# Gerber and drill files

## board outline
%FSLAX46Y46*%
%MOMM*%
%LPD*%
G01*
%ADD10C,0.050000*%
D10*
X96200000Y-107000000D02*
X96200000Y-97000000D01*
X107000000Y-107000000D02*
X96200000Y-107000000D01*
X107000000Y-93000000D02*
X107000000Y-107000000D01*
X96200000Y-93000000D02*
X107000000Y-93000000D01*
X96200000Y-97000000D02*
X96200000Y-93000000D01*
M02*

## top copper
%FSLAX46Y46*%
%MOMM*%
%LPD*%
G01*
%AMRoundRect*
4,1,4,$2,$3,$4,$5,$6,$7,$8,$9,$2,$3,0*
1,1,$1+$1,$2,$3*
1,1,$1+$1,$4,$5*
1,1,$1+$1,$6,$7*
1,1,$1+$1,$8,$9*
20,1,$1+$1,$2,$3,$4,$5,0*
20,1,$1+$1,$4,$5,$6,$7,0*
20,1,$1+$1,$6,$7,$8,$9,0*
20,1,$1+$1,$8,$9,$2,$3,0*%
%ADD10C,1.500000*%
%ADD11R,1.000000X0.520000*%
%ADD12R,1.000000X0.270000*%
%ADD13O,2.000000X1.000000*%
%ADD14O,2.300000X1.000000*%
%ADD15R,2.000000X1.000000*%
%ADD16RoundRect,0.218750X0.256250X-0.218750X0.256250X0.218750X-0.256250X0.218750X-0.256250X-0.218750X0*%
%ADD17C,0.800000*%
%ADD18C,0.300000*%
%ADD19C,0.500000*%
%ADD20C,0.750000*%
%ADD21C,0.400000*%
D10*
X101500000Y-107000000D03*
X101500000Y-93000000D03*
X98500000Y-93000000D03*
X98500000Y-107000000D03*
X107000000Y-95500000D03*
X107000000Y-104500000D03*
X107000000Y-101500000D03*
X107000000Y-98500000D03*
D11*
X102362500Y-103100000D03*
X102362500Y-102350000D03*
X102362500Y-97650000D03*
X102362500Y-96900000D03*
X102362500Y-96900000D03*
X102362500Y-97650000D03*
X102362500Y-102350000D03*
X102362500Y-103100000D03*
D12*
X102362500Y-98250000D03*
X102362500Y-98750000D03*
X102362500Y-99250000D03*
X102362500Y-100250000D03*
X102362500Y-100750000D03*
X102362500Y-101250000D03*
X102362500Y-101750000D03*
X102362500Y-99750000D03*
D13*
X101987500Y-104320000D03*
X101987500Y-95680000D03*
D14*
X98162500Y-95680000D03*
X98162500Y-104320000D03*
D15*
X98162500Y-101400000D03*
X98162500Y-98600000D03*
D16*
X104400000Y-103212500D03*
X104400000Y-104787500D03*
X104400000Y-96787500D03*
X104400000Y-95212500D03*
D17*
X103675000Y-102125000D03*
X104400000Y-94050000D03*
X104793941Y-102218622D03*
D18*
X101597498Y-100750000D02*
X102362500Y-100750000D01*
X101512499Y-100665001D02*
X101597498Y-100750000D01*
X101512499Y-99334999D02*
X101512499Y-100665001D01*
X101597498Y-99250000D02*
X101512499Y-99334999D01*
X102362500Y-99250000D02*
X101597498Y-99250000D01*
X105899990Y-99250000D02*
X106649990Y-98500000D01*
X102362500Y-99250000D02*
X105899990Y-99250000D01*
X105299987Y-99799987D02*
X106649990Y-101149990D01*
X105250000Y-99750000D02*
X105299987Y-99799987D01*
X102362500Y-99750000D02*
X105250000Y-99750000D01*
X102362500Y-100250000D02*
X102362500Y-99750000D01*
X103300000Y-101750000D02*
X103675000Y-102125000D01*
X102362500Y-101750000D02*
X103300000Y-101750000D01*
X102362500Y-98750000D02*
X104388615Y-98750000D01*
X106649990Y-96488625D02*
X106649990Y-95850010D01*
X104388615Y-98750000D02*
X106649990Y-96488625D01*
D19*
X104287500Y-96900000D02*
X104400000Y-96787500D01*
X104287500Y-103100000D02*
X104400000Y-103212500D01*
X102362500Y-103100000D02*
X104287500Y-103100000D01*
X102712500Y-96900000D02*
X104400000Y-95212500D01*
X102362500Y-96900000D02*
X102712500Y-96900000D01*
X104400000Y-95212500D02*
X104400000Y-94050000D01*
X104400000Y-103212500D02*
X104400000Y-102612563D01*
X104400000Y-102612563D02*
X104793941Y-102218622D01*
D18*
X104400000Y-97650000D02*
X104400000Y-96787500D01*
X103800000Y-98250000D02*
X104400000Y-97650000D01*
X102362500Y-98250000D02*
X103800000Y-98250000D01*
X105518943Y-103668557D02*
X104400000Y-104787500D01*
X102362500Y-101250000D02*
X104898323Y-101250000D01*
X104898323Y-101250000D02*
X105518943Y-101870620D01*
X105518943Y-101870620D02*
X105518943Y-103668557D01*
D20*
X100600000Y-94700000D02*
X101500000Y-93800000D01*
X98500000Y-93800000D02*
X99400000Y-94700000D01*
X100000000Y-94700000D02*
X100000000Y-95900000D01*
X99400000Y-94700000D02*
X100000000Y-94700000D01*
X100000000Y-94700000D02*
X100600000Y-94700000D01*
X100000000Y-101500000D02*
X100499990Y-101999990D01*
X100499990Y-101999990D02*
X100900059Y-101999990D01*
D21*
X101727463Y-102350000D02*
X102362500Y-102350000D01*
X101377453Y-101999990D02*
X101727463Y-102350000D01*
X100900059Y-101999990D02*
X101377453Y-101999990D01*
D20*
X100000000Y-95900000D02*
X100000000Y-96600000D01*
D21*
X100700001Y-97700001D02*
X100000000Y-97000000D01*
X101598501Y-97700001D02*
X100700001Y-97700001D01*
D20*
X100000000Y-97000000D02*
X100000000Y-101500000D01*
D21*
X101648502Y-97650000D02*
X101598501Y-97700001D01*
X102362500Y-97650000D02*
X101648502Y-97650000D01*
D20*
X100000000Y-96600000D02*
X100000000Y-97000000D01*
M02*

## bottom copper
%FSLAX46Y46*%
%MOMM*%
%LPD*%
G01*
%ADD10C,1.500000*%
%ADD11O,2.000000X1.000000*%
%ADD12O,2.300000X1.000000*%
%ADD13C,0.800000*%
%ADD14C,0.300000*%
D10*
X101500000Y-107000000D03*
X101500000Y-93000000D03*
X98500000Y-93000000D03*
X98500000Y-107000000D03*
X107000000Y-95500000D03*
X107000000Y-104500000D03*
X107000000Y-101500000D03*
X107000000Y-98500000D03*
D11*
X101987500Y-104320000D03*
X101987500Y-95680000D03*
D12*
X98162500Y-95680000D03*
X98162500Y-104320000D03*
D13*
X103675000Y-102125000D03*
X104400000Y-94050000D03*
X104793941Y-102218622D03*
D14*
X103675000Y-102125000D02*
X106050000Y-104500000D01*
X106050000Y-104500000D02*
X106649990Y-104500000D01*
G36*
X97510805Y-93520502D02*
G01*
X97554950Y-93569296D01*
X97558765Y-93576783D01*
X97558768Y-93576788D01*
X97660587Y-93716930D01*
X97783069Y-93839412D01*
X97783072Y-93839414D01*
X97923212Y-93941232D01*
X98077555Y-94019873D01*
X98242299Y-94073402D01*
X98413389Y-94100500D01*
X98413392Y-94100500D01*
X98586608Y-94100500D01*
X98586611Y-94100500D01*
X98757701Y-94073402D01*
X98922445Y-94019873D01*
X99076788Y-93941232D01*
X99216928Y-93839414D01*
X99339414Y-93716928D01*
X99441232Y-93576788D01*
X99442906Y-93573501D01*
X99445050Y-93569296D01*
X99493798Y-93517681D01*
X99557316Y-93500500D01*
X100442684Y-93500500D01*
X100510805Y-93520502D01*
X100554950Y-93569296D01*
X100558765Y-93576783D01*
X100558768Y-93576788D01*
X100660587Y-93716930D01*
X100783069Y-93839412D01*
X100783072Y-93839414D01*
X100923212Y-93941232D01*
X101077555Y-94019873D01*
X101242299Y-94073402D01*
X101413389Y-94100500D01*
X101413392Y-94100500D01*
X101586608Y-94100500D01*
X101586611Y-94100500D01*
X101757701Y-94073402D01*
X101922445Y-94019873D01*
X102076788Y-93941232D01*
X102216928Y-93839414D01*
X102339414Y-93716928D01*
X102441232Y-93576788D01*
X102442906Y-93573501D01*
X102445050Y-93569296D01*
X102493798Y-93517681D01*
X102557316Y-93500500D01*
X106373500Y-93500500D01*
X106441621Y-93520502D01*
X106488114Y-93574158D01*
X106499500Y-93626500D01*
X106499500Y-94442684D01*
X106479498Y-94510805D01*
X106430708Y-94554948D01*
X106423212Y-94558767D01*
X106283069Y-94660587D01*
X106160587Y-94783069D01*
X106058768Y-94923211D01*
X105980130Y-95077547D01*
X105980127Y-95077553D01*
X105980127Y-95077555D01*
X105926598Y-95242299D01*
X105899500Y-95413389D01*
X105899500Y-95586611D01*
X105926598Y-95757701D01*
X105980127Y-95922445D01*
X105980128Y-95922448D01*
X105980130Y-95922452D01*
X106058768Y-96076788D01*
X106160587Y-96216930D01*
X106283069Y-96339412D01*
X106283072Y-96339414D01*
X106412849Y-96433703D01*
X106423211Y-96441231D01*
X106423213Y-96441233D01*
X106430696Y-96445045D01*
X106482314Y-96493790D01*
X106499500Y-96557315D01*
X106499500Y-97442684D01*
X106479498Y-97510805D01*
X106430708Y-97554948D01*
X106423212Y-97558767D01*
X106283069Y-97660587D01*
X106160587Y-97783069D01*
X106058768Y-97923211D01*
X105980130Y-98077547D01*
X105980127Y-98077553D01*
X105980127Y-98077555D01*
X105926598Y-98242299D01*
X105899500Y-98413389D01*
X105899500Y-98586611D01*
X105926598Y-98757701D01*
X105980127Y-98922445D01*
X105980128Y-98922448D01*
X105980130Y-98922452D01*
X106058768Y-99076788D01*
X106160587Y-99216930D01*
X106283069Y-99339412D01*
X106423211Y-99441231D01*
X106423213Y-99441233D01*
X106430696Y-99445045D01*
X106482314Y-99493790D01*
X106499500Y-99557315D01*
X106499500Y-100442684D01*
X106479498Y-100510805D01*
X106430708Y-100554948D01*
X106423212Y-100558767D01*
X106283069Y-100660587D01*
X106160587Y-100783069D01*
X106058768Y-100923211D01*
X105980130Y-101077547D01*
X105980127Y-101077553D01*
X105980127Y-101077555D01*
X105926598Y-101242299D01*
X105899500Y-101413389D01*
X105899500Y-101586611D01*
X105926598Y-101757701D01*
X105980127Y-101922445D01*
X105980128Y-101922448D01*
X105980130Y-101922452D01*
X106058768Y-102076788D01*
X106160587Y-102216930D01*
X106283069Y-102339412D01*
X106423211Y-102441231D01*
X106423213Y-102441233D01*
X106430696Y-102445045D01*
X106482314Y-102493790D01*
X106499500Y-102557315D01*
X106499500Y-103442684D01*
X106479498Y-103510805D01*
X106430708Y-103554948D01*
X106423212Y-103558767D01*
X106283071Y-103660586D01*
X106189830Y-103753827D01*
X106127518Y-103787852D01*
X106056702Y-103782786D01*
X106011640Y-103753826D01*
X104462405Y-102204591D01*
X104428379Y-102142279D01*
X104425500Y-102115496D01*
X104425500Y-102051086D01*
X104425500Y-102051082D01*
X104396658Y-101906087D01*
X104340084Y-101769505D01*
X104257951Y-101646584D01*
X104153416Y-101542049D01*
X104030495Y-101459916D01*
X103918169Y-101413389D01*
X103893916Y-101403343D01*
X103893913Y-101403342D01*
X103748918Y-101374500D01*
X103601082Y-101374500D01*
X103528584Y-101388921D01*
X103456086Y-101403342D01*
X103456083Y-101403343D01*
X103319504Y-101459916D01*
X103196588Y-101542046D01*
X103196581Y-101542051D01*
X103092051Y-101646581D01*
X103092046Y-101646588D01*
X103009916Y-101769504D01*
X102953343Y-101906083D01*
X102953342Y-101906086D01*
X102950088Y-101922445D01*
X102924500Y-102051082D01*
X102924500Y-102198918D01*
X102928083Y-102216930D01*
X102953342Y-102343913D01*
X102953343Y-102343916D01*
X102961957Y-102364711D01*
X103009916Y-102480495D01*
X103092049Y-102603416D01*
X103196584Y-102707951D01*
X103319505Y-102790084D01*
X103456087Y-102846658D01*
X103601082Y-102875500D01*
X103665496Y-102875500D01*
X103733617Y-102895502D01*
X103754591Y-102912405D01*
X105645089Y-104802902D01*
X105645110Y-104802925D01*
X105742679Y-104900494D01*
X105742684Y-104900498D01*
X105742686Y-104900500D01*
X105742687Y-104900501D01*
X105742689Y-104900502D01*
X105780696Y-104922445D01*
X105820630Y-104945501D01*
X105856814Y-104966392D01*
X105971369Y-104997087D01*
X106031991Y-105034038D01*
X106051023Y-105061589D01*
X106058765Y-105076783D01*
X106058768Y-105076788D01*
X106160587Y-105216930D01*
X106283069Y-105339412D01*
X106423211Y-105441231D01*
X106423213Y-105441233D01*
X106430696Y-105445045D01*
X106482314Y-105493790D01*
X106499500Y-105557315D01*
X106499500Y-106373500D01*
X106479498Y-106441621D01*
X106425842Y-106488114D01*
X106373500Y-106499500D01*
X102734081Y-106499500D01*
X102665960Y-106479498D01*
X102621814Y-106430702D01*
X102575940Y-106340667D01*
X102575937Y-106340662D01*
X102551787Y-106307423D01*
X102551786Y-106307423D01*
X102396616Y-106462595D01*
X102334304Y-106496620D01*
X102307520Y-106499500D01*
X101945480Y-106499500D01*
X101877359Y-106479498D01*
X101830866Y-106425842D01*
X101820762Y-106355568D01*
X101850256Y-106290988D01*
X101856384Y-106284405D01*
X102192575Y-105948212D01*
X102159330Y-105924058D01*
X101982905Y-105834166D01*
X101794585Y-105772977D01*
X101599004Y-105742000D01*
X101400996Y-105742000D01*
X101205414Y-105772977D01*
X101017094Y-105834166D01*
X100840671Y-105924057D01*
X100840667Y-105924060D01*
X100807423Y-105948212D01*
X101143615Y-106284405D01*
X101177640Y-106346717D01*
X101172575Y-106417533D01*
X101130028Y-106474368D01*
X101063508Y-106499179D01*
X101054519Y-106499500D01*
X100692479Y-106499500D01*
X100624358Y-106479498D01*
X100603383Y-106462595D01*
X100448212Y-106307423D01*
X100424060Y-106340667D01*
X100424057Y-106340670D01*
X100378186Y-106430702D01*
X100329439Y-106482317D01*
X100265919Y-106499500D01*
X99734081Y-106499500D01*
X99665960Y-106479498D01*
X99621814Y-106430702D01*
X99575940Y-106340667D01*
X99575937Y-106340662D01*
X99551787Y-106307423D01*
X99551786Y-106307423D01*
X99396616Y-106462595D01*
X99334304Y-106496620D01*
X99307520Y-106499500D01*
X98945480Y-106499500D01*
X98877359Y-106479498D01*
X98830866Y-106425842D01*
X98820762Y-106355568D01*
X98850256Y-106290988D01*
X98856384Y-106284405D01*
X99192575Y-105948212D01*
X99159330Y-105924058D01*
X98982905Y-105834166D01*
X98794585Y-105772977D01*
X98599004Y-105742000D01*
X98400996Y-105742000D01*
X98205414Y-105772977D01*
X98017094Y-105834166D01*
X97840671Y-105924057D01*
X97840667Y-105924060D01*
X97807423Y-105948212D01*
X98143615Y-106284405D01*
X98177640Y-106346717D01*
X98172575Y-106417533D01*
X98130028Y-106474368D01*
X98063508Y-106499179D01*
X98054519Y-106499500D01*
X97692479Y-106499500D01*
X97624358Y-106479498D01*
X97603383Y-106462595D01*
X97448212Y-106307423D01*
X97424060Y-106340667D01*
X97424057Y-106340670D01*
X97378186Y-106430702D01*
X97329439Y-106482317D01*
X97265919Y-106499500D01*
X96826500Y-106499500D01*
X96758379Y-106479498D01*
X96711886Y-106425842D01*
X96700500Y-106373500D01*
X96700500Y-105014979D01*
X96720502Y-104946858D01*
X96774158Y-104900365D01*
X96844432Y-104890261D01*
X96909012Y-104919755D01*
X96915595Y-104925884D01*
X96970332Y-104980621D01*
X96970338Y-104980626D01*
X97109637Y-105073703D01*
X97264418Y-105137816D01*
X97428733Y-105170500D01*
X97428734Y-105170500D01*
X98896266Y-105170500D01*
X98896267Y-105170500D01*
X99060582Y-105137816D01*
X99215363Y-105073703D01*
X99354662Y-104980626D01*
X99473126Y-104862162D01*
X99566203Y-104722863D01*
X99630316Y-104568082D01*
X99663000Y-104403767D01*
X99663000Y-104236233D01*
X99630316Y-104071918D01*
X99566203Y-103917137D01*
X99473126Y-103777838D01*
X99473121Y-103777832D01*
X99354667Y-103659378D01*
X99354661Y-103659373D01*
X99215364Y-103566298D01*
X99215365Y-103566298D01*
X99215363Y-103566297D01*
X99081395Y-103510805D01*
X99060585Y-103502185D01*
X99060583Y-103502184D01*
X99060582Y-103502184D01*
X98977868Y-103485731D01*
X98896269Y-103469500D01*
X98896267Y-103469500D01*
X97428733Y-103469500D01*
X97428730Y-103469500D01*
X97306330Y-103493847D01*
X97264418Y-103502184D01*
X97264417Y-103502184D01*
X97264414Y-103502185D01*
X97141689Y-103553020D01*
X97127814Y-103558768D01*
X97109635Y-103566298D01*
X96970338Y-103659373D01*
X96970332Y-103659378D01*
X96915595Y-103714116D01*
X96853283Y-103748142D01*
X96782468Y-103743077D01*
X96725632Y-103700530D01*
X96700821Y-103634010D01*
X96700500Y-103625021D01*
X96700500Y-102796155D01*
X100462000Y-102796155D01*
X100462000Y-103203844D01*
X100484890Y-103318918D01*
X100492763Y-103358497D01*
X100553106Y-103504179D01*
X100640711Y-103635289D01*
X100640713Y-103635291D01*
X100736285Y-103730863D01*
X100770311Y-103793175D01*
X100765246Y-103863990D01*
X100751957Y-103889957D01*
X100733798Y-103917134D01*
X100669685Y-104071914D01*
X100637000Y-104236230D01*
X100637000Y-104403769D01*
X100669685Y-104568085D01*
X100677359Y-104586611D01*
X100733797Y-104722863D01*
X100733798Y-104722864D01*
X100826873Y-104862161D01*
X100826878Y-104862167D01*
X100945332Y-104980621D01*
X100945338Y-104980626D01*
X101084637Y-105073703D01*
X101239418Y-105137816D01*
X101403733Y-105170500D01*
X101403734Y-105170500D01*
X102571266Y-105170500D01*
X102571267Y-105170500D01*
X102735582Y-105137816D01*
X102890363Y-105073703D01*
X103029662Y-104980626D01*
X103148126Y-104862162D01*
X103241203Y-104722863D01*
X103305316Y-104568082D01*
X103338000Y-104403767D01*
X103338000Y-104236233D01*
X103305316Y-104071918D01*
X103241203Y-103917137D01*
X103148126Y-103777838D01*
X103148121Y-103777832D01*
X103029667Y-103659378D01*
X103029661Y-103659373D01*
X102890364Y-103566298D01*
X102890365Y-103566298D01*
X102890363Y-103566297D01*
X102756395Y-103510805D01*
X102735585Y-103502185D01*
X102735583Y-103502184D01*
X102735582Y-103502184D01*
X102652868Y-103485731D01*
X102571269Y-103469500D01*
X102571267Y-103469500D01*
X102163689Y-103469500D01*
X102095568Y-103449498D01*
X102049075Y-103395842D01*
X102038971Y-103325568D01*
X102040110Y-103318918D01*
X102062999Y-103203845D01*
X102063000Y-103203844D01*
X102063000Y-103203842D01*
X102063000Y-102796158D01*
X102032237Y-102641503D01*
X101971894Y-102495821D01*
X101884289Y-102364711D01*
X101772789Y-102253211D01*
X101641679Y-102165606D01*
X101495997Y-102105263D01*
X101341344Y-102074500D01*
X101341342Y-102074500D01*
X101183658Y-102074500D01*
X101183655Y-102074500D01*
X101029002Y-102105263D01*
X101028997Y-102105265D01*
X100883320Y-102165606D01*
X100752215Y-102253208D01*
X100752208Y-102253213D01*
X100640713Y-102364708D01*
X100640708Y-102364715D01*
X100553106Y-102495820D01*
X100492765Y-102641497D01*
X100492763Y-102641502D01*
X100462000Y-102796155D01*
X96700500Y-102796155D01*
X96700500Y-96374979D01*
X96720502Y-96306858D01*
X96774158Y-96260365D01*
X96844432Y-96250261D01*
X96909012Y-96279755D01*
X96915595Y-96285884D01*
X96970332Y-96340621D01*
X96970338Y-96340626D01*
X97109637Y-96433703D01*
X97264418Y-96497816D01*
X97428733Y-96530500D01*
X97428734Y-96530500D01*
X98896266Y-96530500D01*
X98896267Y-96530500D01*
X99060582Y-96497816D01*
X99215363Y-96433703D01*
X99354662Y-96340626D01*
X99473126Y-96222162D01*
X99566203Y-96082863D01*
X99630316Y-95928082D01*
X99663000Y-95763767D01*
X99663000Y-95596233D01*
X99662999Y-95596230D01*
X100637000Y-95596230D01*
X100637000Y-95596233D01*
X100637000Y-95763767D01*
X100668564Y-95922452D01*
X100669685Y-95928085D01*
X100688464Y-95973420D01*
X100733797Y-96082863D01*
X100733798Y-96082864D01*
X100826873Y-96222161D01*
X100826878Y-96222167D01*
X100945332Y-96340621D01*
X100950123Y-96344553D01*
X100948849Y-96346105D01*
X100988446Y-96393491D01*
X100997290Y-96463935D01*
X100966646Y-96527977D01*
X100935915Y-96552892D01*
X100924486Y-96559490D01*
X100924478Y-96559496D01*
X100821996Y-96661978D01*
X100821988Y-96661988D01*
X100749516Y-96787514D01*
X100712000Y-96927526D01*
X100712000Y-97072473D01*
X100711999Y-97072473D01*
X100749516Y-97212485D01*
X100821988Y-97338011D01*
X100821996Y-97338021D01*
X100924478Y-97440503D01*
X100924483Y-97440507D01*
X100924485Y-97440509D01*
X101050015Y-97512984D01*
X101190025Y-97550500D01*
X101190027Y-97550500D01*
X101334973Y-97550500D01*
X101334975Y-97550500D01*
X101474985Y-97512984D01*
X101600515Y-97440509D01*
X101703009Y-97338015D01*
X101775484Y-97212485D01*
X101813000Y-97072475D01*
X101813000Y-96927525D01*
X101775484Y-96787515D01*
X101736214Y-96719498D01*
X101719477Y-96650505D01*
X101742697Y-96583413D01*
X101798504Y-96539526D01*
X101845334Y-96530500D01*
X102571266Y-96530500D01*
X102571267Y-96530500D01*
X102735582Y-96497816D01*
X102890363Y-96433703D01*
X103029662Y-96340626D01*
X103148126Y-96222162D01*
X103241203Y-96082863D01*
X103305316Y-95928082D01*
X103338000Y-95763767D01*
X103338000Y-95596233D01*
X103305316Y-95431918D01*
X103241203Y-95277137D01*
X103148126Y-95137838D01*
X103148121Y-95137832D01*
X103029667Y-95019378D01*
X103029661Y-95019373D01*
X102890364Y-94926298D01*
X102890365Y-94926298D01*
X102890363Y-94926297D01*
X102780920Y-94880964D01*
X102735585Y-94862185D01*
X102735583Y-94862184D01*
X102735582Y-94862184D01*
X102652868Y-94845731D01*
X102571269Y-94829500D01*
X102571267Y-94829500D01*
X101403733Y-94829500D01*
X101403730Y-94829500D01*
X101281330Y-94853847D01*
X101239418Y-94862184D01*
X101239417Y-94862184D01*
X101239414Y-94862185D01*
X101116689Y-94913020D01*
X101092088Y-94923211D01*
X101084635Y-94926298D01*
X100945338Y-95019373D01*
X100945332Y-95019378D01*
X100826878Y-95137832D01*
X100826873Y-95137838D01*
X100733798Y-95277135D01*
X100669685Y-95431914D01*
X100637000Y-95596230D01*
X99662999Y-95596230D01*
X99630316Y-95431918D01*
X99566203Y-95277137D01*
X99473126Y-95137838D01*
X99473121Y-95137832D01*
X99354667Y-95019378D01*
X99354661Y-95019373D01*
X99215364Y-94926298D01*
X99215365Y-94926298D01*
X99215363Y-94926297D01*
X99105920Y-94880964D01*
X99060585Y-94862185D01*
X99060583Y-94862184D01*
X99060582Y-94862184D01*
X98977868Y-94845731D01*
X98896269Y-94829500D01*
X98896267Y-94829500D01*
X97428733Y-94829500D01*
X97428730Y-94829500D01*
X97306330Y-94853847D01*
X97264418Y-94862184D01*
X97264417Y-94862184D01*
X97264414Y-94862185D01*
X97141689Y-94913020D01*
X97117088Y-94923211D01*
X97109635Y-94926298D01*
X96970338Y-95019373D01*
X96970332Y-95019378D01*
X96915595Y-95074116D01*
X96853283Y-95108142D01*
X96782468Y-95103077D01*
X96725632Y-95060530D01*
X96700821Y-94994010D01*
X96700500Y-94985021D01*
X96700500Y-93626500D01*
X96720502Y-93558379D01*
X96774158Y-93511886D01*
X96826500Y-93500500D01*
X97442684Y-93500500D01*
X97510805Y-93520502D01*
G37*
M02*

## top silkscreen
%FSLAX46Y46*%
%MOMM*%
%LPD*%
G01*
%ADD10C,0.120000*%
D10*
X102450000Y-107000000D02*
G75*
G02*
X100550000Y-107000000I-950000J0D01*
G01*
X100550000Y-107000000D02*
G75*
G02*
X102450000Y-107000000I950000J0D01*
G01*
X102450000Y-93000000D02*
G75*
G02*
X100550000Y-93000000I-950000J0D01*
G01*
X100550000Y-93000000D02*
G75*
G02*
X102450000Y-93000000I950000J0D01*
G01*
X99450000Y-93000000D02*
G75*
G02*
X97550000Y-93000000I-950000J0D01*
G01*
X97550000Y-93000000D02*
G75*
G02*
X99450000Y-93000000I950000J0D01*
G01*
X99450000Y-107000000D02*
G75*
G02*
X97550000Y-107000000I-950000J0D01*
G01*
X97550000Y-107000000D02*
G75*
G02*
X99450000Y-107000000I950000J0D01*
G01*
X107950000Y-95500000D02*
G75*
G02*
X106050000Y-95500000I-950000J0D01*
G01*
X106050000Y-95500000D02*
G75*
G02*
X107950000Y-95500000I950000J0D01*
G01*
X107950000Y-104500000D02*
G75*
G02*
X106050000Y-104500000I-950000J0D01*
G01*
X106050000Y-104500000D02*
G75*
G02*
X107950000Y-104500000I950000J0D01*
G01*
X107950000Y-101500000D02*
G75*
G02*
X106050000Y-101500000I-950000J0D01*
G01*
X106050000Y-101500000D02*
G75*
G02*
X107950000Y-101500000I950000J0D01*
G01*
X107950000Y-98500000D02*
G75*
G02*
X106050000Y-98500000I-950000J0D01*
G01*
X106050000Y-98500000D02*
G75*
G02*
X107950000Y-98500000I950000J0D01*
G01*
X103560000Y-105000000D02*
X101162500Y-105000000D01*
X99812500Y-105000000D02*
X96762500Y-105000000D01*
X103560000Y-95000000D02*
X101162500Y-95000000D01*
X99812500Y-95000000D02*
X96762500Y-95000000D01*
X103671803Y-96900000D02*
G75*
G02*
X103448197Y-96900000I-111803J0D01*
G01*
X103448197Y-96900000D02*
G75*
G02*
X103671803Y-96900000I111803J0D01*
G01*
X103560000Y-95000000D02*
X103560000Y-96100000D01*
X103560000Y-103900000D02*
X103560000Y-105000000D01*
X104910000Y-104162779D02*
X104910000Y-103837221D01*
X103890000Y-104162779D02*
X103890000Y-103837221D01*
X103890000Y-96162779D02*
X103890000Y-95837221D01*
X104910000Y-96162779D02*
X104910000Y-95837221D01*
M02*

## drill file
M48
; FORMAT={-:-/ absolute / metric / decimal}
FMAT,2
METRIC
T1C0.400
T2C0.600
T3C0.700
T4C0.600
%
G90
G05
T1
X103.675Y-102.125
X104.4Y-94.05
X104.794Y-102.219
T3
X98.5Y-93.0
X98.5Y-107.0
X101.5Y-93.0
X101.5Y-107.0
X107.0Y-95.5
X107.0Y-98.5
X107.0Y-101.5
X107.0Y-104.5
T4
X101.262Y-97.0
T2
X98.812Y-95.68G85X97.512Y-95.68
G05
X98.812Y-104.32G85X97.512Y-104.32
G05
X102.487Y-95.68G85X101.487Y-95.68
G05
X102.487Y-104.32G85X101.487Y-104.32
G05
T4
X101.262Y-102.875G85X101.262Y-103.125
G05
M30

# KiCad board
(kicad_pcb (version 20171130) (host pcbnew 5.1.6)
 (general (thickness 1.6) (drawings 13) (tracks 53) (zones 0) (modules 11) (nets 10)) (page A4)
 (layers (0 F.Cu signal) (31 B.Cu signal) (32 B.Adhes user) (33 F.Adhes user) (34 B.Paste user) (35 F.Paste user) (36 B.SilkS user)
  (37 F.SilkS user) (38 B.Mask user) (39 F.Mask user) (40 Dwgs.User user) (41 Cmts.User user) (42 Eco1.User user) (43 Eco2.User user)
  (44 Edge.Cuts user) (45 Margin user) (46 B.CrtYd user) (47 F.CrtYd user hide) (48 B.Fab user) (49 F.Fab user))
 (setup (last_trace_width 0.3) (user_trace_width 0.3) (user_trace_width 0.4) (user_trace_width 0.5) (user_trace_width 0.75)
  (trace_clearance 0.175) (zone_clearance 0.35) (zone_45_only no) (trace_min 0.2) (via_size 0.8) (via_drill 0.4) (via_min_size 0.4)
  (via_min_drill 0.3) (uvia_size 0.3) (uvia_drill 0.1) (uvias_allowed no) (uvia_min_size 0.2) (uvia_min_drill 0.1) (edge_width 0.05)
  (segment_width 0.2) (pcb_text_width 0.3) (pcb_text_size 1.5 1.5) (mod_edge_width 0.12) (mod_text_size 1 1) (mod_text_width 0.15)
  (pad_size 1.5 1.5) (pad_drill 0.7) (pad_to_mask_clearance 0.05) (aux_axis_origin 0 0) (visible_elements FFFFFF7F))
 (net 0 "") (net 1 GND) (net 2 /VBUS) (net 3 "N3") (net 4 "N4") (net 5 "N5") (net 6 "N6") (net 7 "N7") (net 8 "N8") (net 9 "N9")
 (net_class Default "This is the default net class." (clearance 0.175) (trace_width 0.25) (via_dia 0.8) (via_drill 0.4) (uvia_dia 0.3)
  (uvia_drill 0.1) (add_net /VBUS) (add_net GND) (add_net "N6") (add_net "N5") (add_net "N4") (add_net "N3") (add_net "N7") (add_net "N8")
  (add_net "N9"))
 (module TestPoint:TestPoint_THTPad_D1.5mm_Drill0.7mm (layer F.Cu) (at 101.5 107) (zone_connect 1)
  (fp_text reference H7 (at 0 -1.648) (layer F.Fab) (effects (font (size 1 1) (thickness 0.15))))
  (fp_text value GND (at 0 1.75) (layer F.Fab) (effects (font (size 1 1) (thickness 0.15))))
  (fp_circle (center 0 0) (end 0 0.95) (layer F.SilkS) (width 0.12))
  (pad 1 thru_hole circle (at 0 0) (size 1.5 1.5) (drill 0.7) (layers *.Cu *.Mask) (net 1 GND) (zone_connect 1)))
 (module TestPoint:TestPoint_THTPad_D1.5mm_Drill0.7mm (layer F.Cu) (at 101.5 93)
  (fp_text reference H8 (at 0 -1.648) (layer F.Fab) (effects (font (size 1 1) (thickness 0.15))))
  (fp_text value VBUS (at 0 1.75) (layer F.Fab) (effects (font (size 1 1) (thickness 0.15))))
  (fp_circle (center 0 0) (end 0 0.95) (layer F.SilkS) (width 0.12))
  (pad 1 thru_hole circle (at 0 0) (size 1.5 1.5) (drill 0.7) (layers *.Cu *.Mask) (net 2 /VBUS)))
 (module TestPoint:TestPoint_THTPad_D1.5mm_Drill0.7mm (layer F.Cu) (at 98.5 93)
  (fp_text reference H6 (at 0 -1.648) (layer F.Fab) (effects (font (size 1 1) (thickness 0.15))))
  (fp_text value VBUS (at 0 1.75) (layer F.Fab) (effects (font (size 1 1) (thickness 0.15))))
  (fp_circle (center 0 0) (end 0 0.95) (layer F.SilkS) (width 0.12))
  (pad 1 thru_hole circle (at 0 0) (size 1.5 1.5) (drill 0.7) (layers *.Cu *.Mask) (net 2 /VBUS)))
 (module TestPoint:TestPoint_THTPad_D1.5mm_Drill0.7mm (layer F.Cu) (at 98.5 107) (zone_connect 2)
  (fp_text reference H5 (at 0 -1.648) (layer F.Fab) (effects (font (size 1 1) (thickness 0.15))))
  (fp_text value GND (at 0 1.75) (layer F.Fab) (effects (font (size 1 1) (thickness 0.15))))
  (fp_circle (center 0 0) (end 0 0.95) (layer F.SilkS) (width 0.12))
  (pad 1 thru_hole circle (at 0 0) (size 1.5 1.5) (drill 0.7) (layers *.Cu *.Mask) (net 1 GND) (zone_connect 1)))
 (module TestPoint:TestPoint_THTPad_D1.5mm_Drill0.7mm (layer F.Cu) (at 107 95.5)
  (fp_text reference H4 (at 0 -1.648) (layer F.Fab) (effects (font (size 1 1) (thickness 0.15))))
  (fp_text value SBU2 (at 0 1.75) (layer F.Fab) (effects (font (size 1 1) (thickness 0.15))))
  (fp_circle (center 0 0) (end 0 0.95) (layer F.SilkS) (width 0.12))
  (pad 1 thru_hole circle (at 0 0) (size 1.5 1.5) (drill 0.7) (layers *.Cu *.Mask) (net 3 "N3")))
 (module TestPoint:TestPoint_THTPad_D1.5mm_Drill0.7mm (layer F.Cu) (at 107 104.5)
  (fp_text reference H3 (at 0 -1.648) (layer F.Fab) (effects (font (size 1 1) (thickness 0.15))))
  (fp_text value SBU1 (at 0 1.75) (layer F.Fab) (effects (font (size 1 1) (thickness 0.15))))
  (fp_circle (center 0 0) (end 0 0.95) (layer F.SilkS) (width 0.12))
  (pad 1 thru_hole circle (at 0 0) (size 1.5 1.5) (drill 0.7) (layers *.Cu *.Mask) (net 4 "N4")))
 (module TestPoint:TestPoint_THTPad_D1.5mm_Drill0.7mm (layer F.Cu) (at 107 101.5)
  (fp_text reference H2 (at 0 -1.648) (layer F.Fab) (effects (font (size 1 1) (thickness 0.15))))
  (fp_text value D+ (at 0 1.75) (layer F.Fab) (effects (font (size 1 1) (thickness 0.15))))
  (fp_circle (center 0 0) (end 0 0.95) (layer F.SilkS) (width 0.12))
  (pad 1 thru_hole circle (at 0 0) (size 1.5 1.5) (drill 0.7) (layers *.Cu *.Mask) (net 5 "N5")))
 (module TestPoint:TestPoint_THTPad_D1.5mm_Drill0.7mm (layer F.Cu) (at 107 98.5)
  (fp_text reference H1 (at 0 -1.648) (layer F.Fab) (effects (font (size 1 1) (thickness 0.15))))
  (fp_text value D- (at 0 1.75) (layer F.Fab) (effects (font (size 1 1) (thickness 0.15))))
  (fp_circle (center 0 0) (end 0 0.95) (layer F.SilkS) (width 0.12))
  (pad 1 thru_hole circle (at 0 0) (size 1.5 1.5) (drill 0.7) (layers *.Cu *.Mask) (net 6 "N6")))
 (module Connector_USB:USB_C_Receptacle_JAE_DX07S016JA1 (layer F.Cu) (at 100 100 270)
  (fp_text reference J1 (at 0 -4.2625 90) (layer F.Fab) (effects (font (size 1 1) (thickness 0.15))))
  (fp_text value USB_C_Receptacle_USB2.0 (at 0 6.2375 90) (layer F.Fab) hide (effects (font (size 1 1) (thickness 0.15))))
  (fp_line (start 5 -3.56) (end 5 -1.1625) (layer F.SilkS) (width 0.12))
  (fp_line (start 5 0.1875) (end 5 3.2375) (layer F.SilkS) (width 0.12))
  (fp_line (start -5 -3.56) (end -5 -1.1625) (layer F.SilkS) (width 0.12))
  (fp_line (start -5 0.1875) (end -5 3.2375) (layer F.SilkS) (width 0.12))
  (fp_circle (center -3.1 -3.56) (end -2.988197 -3.56) (layer F.SilkS) (width 0.12))
  (fp_line (start -5 -3.56) (end -3.9 -3.56) (layer F.SilkS) (width 0.12))
  (fp_line (start 3.9 -3.56) (end 5 -3.56) (layer F.SilkS) (width 0.12))
  (pad B1 smd rect (at 3.1 -2.3625 270) (size 0.52 1) (layers F.Cu F.Paste F.Mask) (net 1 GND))
  (pad A9 smd rect (at 2.35 -2.3625 270) (size 0.52 1) (layers F.Cu F.Paste F.Mask) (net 2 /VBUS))
  (pad B9 smd rect (at -2.35 -2.3625 270) (size 0.52 1) (layers F.Cu F.Paste F.Mask) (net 2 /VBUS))
  (pad B12 smd rect (at -3.1 -2.3625 270) (size 0.52 1) (layers F.Cu F.Paste F.Mask) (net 1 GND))
  (pad A1 smd rect (at -3.1 -2.3625 270) (size 0.52 1) (layers F.Cu F.Paste F.Mask) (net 1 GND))
  (pad A4 smd rect (at -2.35 -2.3625 270) (size 0.52 1) (layers F.Cu F.Paste F.Mask) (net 2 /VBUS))
  (pad B4 smd rect (at 2.35 -2.3625 270) (size 0.52 1) (layers F.Cu F.Paste F.Mask) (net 2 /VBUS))
  (pad A12 smd rect (at 3.1 -2.3625 270) (size 0.52 1) (layers F.Cu F.Paste F.Mask) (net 1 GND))
  (pad A5 smd rect (at -1.75 -2.3625 270) (size 0.27 1) (layers F.Cu F.Paste F.Mask) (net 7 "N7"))
  (pad B8 smd rect (at -1.25 -2.3625 270) (size 0.27 1) (layers F.Cu F.Paste F.Mask) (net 3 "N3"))
  (pad B7 smd rect (at -0.75 -2.3625 270) (size 0.27 1) (layers F.Cu F.Paste F.Mask) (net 6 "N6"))
  (pad B6 smd rect (at 0.25 -2.3625 270) (size 0.27 1) (layers F.Cu F.Paste F.Mask) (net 5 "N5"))
  (pad A7 smd rect (at 0.75 -2.3625 270) (size 0.27 1) (layers F.Cu F.Paste F.Mask) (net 6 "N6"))
  (pad B5 smd rect (at 1.25 -2.3625 270) (size 0.27 1) (layers F.Cu F.Paste F.Mask) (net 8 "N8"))
  (pad A8 smd rect (at 1.75 -2.3625 270) (size 0.27 1) (layers F.Cu F.Paste F.Mask) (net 4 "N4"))
  (pad A6 smd rect (at -0.25 -2.3625 270) (size 0.27 1) (layers F.Cu F.Paste F.Mask) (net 5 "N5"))
  (pad S1 thru_hole oval (at 4.32 -1.9875 270) (size 1 2) (drill oval 0.6 1.6) (layers *.Cu *.Mask) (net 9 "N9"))
  (pad S1 thru_hole oval (at -4.32 -1.9875 270) (size 1 2) (drill oval 0.6 1.6) (layers *.Cu *.Mask) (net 9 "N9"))
  (pad "" np_thru_hole circle (at -3 -1.2625 270) (size 0.6 0.6) (drill 0.6) (layers *.Cu *.Mask))
  (pad S1 thru_hole oval (at -4.32 1.8375 270) (size 1 2.3) (drill oval 0.6 1.9) (layers *.Cu *.Mask) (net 9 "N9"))
  (pad "" np_thru_hole oval (at 3 -1.2625 270) (size 0.85 0.6) (drill oval 0.85 0.6) (layers *.Cu *.Mask))
  (pad S1 thru_hole oval (at 4.32 1.8375 270) (size 1 2.3) (drill oval 0.6 1.9) (layers *.Cu *.Mask) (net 9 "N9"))
  (pad S1 smd rect (at 1.4 1.8375 270) (size 1 2) (layers F.Cu F.Paste F.Mask) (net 9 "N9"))
  (pad S1 smd rect (at -1.4 1.8375 270) (size 1 2) (layers F.Cu F.Paste F.Mask) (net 9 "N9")))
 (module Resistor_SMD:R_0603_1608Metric (layer F.Cu) (at 104.4 104 90)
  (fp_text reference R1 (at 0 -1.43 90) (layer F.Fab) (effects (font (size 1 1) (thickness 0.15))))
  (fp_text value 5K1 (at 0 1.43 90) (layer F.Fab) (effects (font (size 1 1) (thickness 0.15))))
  (fp_line (start -0.162779 0.51) (end 0.162779 0.51) (layer F.SilkS) (width 0.12))
  (fp_line (start -0.162779 -0.51) (end 0.162779 -0.51) (layer F.SilkS) (width 0.12))
  (pad 2 smd roundrect (at 0.7875 0 90) (size 0.875 0.95) (layers F.Cu F.Paste F.Mask) (roundrect_rratio 0.25) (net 1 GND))
  (pad 1 smd roundrect (at -0.7875 0 90) (size 0.875 0.95) (layers F.Cu F.Paste F.Mask) (roundrect_rratio 0.25) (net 8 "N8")))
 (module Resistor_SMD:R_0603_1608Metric (layer F.Cu) (at 104.4 96 90)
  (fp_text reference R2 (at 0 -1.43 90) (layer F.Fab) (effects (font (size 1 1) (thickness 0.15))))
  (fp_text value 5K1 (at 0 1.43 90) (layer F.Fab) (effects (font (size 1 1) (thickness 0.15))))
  (fp_line (start -0.162779 -0.51) (end 0.162779 -0.51) (layer F.SilkS) (width 0.12))
  (fp_line (start -0.162779 0.51) (end 0.162779 0.51) (layer F.SilkS) (width 0.12))
  (pad 1 smd roundrect (at -0.7875 0 90) (size 0.875 0.95) (layers F.Cu F.Paste F.Mask) (roundrect_rratio 0.25) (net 7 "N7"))
  (pad 2 smd roundrect (at 0.7875 0 90) (size 0.875 0.95) (layers F.Cu F.Paste F.Mask) (roundrect_rratio 0.25) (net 1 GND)))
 (gr_line (start 96.2 107) (end 96.2 97) (layer Edge.Cuts) (width 0.05))
 (gr_line (start 107 107) (end 96.2 107) (layer Edge.Cuts) (width 0.05))
 (gr_line (start 107 93) (end 107 107) (layer Edge.Cuts) (width 0.05))
 (gr_line (start 96.2 93) (end 107 93) (layer Edge.Cuts) (width 0.05))
 (gr_line (start 96.2 97) (end 96.2 93) (layer Edge.Cuts) (width 0.05))
 (segment (start 101.597498 100.75) (end 102.3625 100.75) (width 0.3) (layer F.Cu) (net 6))
 (segment (start 101.512499 100.665001) (end 101.597498 100.75) (width 0.3) (layer F.Cu) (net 6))
 (segment (start 101.512499 99.334999) (end 101.512499 100.665001) (width 0.3) (layer F.Cu) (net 6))
 (segment (start 101.597498 99.25) (end 101.512499 99.334999) (width 0.3) (layer F.Cu) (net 6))
 (segment (start 102.3625 99.25) (end 101.597498 99.25) (width 0.3) (layer F.Cu) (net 6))
 (segment (start 105.89999 99.25) (end 106.64999 98.5) (width 0.3) (layer F.Cu) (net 6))
 (segment (start 102.3625 99.25) (end 105.89999 99.25) (width 0.3) (layer F.Cu) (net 6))
 (segment (start 105.299987 99.799987) (end 106.64999 101.14999) (width 0.3) (layer F.Cu) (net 5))
 (segment (start 105.25 99.75) (end 105.299987 99.799987) (width 0.3) (layer F.Cu) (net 5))
 (segment (start 102.3625 99.75) (end 105.25 99.75) (width 0.3) (layer F.Cu) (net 5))
 (segment (start 102.3625 100.25) (end 102.3625 99.75) (width 0.3) (layer F.Cu) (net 5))
 (via (at 103.675 102.125) (size 0.8) (drill 0.4) (layers F.Cu B.Cu) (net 4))
 (segment (start 103.3 101.75) (end 103.675 102.125) (width 0.3) (layer F.Cu) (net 4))
 (segment (start 102.3625 101.75) (end 103.3 101.75) (width 0.3) (layer F.Cu) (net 4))
 (segment (start 103.675 102.125) (end 106.05 104.5) (width 0.3) (layer B.Cu) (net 4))
 (segment (start 106.05 104.5) (end 106.64999 104.5) (width 0.3) (layer B.Cu) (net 4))
 (segment (start 102.3625 98.75) (end 104.388615 98.75) (width 0.3) (layer F.Cu) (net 3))
 (segment (start 106.64999 96.488625) (end 106.64999 95.85001) (width 0.3) (layer F.Cu) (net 3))
 (segment (start 104.388615 98.75) (end 106.64999 96.488625) (width 0.3) (layer F.Cu) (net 3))
 (segment (start 104.2875 96.9) (end 104.4 96.7875) (width 0.5) (layer F.Cu) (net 7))
 (segment (start 104.2875 103.1) (end 104.4 103.2125) (width 0.5) (layer F.Cu) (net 1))
 (segment (start 102.3625 103.1) (end 104.2875 103.1) (width 0.5) (layer F.Cu) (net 1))
 (segment (start 102.7125 96.9) (end 104.4 95.2125) (width 0.5) (layer F.Cu) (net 1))
 (segment (start 102.3625 96.9) (end 102.7125 96.9) (width 0.5) (layer F.Cu) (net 1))
 (via (at 104.4 94.05) (size 0.8) (drill 0.4) (layers F.Cu B.Cu) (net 1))
 (segment (start 104.4 95.2125) (end 104.4 94.05) (width 0.5) (layer F.Cu) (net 1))
 (via (at 104.793941 102.218622) (size 0.8) (drill 0.4) (layers F.Cu B.Cu) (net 1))
 (segment (start 104.4 103.2125) (end 104.4 102.612563) (width 0.5) (layer F.Cu) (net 1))
 (segment (start 104.4 102.612563) (end 104.793941 102.218622) (width 0.5) (layer F.Cu) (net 1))
 (segment (start 104.4 97.65) (end 104.4 96.7875) (width 0.3) (layer F.Cu) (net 7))
 (segment (start 103.8 98.25) (end 104.4 97.65) (width 0.3) (layer F.Cu) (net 7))
 (segment (start 102.3625 98.25) (end 103.8 98.25) (width 0.3) (layer F.Cu) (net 7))
 (segment (start 105.518943 103.668557) (end 104.4 104.7875) (width 0.3) (layer F.Cu) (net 8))
 (segment (start 102.3625 101.25) (end 104.898323 101.25) (width 0.3) (layer F.Cu) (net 8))
 (segment (start 104.898323 101.25) (end 105.518943 101.87062) (width 0.3) (layer F.Cu) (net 8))
 (segment (start 105.518943 101.87062) (end 105.518943 103.668557) (width 0.3) (layer F.Cu) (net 8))
 (segment (start 100.6 94.7) (end 101.5 93.8) (width 0.75) (layer F.Cu) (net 2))
 (segment (start 98.5 93.8) (end 99.4 94.7) (width 0.75) (layer F.Cu) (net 2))
 (segment (start 100 94.7) (end 100 95.9) (width 0.75) (layer F.Cu) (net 2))
 (segment (start 99.4 94.7) (end 100 94.7) (width 0.75) (layer F.Cu) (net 2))
 (segment (start 100 94.7) (end 100.6 94.7) (width 0.75) (layer F.Cu) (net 2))
 (segment (start 100 101.5) (end 100.49999 101.99999) (width 0.75) (layer F.Cu) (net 2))
 (segment (start 100.49999 101.99999) (end 100.900059 101.99999) (width 0.75) (layer F.Cu) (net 2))
 (segment (start 101.727463 102.35) (end 102.3625 102.35) (width 0.4) (layer F.Cu) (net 2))
 (segment (start 101.377453 101.99999) (end 101.727463 102.35) (width 0.4) (layer F.Cu) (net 2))
 (segment (start 100.900059 101.99999) (end 101.377453 101.99999) (width 0.4) (layer F.Cu) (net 2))
 (segment (start 100 95.9) (end 100 96.6) (width 0.75) (layer F.Cu) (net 2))
 (segment (start 100.700001 97.700001) (end 100 97) (width 0.4) (layer F.Cu) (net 2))
 (segment (start 101.598501 97.700001) (end 100.700001 97.700001) (width 0.4) (layer F.Cu) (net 2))
 (segment (start 100 97) (end 100 101.5) (width 0.75) (layer F.Cu) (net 2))
 (segment (start 101.648502 97.65) (end 101.598501 97.700001) (width 0.4) (layer F.Cu) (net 2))
 (segment (start 102.3625 97.65) (end 101.648502 97.65) (width 0.4) (layer F.Cu) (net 2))
 (segment (start 100 96.6) (end 100 97) (width 0.75) (layer F.Cu) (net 2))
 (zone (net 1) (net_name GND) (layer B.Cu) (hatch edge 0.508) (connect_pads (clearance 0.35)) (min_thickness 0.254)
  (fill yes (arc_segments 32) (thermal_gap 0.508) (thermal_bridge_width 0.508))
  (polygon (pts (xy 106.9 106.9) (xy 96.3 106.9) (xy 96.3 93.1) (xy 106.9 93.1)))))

